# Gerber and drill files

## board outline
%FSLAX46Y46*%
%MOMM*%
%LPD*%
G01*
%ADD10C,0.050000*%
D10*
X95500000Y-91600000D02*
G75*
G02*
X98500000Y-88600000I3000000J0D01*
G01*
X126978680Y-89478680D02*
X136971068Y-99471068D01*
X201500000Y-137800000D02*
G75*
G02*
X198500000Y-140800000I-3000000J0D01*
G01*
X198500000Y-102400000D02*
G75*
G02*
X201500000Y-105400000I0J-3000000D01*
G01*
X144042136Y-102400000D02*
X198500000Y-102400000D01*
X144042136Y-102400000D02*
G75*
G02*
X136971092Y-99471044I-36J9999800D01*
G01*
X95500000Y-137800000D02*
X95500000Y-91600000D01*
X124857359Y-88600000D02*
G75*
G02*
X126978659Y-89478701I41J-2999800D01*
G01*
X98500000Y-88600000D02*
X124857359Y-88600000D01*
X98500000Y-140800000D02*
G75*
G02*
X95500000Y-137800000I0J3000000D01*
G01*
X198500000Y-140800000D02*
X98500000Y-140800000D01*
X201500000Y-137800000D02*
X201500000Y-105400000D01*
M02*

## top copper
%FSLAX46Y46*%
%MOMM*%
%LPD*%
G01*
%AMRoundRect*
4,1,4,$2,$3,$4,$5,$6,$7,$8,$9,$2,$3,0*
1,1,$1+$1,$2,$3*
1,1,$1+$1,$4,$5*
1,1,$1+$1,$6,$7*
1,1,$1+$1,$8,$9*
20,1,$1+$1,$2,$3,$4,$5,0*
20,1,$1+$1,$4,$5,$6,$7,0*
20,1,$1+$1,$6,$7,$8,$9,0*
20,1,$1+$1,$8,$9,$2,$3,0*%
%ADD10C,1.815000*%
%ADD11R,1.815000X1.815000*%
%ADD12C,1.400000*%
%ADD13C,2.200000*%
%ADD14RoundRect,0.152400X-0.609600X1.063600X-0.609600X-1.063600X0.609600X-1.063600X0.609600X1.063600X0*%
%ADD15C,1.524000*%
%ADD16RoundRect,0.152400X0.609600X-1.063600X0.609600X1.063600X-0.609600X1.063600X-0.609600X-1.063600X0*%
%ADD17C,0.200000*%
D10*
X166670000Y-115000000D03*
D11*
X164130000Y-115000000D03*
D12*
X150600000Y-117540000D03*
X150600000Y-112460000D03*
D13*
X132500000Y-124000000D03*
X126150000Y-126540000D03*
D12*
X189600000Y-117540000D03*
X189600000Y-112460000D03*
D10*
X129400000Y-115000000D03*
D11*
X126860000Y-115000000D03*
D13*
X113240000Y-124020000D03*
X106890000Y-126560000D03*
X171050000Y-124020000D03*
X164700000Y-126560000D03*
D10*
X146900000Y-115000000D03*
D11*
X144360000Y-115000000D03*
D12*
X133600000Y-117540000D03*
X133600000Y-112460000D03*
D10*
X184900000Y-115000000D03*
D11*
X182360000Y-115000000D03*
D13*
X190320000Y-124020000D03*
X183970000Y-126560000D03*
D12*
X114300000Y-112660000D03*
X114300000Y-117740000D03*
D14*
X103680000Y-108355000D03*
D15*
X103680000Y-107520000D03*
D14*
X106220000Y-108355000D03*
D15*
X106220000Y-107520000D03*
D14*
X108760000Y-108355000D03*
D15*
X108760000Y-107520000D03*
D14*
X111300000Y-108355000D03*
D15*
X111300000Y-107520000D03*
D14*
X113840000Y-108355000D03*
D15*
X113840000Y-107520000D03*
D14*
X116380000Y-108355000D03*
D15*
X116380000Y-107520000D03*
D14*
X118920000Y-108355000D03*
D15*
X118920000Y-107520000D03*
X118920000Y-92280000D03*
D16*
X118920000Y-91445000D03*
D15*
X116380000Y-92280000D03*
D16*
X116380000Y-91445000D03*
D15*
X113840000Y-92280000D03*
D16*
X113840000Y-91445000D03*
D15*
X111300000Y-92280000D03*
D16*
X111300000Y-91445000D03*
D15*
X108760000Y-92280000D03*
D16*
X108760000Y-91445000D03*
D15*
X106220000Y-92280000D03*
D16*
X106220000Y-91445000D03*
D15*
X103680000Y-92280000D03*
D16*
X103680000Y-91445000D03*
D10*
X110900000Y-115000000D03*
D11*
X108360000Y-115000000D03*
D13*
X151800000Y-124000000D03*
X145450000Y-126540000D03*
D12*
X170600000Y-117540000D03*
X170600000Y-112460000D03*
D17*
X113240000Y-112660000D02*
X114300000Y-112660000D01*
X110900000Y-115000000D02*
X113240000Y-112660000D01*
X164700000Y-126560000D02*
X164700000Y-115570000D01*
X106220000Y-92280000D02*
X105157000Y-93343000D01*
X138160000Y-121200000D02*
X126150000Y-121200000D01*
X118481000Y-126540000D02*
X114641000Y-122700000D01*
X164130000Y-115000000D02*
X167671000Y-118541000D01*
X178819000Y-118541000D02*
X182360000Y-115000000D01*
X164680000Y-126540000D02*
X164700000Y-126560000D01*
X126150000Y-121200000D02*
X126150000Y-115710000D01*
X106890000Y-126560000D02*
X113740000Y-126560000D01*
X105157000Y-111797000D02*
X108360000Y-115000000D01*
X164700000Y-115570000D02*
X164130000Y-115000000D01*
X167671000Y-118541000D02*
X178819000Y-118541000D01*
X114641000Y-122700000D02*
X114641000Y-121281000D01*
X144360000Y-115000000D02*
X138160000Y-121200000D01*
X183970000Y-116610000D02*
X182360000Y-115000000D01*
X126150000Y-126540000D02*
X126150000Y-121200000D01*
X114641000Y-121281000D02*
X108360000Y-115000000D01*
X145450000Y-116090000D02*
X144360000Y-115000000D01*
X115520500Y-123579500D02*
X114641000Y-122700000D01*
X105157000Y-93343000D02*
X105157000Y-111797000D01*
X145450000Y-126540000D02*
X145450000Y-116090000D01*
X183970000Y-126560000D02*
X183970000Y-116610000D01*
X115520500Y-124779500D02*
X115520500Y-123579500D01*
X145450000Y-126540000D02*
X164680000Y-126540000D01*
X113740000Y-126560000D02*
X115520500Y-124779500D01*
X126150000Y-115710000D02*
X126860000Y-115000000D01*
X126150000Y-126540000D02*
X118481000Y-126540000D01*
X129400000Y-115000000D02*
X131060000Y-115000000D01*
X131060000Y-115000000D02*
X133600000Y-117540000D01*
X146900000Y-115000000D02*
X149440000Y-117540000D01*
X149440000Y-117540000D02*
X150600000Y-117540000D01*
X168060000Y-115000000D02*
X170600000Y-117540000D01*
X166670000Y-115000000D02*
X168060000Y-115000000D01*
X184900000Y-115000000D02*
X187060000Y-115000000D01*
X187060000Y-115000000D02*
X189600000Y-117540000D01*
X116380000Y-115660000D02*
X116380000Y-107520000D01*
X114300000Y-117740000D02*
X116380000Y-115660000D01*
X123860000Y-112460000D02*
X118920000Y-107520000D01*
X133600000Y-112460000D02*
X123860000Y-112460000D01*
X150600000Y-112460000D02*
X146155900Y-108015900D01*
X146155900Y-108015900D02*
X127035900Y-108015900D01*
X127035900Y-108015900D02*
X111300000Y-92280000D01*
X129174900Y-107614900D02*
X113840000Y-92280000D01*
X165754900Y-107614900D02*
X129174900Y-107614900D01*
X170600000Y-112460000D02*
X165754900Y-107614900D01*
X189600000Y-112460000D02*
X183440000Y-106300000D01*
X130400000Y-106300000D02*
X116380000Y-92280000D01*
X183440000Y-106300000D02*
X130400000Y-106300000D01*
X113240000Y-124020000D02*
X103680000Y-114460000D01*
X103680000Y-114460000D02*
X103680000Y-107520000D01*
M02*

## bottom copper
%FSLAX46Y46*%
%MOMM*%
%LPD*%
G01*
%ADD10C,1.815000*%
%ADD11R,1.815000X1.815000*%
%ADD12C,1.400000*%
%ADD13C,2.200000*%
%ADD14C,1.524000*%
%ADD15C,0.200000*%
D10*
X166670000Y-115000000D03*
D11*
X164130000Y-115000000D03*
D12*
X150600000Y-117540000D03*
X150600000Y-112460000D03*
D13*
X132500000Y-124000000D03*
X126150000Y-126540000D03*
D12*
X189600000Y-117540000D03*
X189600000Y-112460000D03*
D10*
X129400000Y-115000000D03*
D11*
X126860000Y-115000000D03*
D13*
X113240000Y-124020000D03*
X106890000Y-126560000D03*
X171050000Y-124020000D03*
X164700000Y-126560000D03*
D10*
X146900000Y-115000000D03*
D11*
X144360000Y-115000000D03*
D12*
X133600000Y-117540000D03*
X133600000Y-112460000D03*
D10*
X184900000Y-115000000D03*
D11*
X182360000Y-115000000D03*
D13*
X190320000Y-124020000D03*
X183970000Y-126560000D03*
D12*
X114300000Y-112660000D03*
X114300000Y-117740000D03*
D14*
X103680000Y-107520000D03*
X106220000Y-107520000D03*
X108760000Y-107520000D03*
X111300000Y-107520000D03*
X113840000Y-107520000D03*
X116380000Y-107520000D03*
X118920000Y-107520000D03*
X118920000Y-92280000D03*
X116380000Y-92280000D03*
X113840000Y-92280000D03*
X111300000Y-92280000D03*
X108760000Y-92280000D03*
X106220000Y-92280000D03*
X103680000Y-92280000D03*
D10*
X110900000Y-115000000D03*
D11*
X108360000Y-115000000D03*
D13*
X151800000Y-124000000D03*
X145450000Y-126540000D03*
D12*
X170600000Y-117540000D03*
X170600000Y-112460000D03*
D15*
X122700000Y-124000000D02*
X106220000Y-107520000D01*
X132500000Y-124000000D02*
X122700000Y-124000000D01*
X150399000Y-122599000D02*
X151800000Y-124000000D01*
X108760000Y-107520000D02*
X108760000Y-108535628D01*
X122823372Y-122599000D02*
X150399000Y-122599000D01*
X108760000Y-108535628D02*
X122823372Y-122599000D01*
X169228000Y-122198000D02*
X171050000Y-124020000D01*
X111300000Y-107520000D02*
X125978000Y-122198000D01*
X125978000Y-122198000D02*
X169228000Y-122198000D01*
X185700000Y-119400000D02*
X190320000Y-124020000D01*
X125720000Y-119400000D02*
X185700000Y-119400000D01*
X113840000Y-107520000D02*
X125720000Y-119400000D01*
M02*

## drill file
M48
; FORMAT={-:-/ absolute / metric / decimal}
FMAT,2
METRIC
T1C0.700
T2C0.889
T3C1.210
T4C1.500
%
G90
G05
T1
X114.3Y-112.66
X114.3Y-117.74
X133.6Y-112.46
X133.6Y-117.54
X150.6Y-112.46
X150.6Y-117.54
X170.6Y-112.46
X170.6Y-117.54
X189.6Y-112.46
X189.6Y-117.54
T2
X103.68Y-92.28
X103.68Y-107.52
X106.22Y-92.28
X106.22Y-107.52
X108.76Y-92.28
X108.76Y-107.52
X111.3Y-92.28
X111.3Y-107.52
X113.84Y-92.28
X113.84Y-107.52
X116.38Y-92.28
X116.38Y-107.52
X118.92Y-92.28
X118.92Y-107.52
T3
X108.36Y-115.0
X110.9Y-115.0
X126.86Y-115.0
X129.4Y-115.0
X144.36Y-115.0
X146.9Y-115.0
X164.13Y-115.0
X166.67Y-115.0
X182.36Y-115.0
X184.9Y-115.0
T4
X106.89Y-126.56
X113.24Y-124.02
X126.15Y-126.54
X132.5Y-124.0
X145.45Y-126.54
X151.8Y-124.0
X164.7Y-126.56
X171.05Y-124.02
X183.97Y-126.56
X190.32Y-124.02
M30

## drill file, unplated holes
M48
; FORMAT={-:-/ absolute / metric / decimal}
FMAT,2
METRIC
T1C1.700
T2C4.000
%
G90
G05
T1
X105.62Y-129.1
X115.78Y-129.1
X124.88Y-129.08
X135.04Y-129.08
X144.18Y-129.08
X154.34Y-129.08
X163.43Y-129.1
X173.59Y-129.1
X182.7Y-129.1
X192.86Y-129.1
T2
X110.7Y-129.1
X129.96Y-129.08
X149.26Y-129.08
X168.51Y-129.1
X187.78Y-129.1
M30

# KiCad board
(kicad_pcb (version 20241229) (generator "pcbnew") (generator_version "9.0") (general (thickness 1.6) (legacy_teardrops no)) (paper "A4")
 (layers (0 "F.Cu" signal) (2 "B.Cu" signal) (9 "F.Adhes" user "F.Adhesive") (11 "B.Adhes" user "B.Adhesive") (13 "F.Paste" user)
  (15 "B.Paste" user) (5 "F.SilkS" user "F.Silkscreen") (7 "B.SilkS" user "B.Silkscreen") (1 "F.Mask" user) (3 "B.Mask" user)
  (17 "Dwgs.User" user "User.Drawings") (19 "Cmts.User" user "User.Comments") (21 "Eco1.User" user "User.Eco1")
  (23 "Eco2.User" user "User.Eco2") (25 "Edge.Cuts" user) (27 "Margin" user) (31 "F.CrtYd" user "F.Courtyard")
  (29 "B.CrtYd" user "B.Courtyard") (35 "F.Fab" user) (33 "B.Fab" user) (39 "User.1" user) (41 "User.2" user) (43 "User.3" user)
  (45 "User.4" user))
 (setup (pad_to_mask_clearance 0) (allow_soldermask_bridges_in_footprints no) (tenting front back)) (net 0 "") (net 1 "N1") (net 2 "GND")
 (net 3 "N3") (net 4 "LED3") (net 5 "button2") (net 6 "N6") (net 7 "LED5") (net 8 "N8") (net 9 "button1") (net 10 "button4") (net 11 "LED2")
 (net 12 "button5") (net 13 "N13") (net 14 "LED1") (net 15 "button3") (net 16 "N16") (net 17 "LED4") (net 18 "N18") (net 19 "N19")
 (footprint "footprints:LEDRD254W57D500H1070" (layer "F.Cu") (at 165.4 115)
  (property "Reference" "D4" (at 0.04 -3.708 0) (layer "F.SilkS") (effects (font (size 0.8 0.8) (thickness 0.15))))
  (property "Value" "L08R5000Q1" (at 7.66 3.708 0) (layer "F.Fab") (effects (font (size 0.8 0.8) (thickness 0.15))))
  (pad "A" thru_hole circle (at 1.27 0) (size 1.815 1.815) (drill 1.21) (layers "*.Cu" "*.Mask") (remove_unused_layers no) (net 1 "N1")
   (solder_mask_margin 0.102))
  (pad "C" thru_hole rect (at -1.27 0) (size 1.815 1.815) (drill 1.21) (layers "*.Cu" "*.Mask") (remove_unused_layers no) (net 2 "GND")
   (solder_mask_margin 0.102)))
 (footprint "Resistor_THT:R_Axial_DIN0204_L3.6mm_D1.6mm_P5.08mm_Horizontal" (layer "F.Cu") (at 150.6 117.54 90)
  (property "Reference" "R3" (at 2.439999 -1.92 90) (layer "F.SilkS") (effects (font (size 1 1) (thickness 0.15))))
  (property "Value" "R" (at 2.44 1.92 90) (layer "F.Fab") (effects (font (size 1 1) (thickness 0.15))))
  (pad "1" thru_hole circle (at 0 0 90) (size 1.4 1.4) (drill 0.7) (layers "*.Cu" "*.Mask") (remove_unused_layers no) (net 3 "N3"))
  (pad "2" thru_hole circle (at 5.08 0 90) (size 1.4 1.4) (drill 0.7) (layers "*.Cu" "*.Mask") (remove_unused_layers no) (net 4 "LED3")))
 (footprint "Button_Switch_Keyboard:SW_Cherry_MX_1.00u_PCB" (layer "F.Cu") (at 132.5 124)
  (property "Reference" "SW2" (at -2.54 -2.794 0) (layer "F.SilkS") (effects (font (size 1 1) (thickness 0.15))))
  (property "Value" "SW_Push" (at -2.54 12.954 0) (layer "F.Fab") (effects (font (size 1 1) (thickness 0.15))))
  (pad "" np_thru_hole circle (at -7.62 5.08) (size 1.7 1.7) (drill 1.7) (layers "*.Cu" "*.Mask"))
  (pad "" np_thru_hole circle (at -2.54 5.08) (size 4 4) (drill 4) (layers "*.Cu" "*.Mask"))
  (pad "" np_thru_hole circle (at 2.54 5.08) (size 1.7 1.7) (drill 1.7) (layers "*.Cu" "*.Mask"))
  (pad "1" thru_hole circle (at 0 0) (size 2.2 2.2) (drill 1.5) (layers "*.Cu" "*.Mask") (remove_unused_layers no) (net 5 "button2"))
  (pad "2" thru_hole circle (at -6.35 2.54) (size 2.2 2.2) (drill 1.5) (layers "*.Cu" "*.Mask") (remove_unused_layers no) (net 2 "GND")))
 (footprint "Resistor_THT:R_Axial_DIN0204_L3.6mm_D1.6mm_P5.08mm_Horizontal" (layer "F.Cu") (at 189.6 117.54 90)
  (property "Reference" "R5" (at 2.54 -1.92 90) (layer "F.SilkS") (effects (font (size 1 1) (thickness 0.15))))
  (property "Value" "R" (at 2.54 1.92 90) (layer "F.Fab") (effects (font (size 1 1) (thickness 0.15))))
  (pad "1" thru_hole circle (at 0 0 90) (size 1.4 1.4) (drill 0.7) (layers "*.Cu" "*.Mask") (remove_unused_layers no) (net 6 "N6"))
  (pad "2" thru_hole circle (at 5.08 0 90) (size 1.4 1.4) (drill 0.7) (layers "*.Cu" "*.Mask") (remove_unused_layers no) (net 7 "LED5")))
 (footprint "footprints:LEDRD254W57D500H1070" (layer "F.Cu") (at 128.13 115)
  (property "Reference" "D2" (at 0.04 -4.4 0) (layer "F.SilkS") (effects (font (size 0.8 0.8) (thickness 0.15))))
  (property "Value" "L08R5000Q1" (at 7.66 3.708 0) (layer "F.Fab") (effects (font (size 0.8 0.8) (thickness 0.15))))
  (pad "A" thru_hole circle (at 1.27 0) (size 1.815 1.815) (drill 1.21) (layers "*.Cu" "*.Mask") (remove_unused_layers no) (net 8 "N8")
   (solder_mask_margin 0.102))
  (pad "C" thru_hole rect (at -1.27 0) (size 1.815 1.815) (drill 1.21) (layers "*.Cu" "*.Mask") (remove_unused_layers no) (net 2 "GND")
   (solder_mask_margin 0.102)))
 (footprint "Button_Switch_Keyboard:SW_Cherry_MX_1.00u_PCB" (layer "F.Cu") (at 113.24 124.02)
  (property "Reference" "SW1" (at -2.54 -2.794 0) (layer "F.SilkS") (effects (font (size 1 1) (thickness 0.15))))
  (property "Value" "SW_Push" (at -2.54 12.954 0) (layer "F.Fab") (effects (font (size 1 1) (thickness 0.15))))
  (pad "" np_thru_hole circle (at -7.62 5.08) (size 1.7 1.7) (drill 1.7) (layers "*.Cu" "*.Mask"))
  (pad "" np_thru_hole circle (at -2.54 5.08) (size 4 4) (drill 4) (layers "*.Cu" "*.Mask"))
  (pad "" np_thru_hole circle (at 2.54 5.08) (size 1.7 1.7) (drill 1.7) (layers "*.Cu" "*.Mask"))
  (pad "1" thru_hole circle (at 0 0) (size 2.2 2.2) (drill 1.5) (layers "*.Cu" "*.Mask") (remove_unused_layers no) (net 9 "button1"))
  (pad "2" thru_hole circle (at -6.35 2.54) (size 2.2 2.2) (drill 1.5) (layers "*.Cu" "*.Mask") (remove_unused_layers no) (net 2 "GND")))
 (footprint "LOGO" (layer "F.Cu") (at 194.1 109.1)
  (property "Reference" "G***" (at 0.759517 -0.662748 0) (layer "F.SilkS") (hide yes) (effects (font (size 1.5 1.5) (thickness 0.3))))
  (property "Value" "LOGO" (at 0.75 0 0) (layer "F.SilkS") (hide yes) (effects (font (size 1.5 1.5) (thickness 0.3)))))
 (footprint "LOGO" (layer "F.Cu") (at 132.976092 101.625741 -30)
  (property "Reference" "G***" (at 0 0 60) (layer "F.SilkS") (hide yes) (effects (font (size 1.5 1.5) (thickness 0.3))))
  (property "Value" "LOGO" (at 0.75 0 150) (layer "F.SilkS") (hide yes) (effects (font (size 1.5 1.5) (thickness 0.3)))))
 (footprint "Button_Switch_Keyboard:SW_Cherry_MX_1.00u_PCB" (layer "F.Cu") (at 171.05 124.02)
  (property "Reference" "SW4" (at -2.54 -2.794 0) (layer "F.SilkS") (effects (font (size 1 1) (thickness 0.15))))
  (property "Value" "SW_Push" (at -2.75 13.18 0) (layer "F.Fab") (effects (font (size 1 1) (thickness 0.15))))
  (pad "" np_thru_hole circle (at -7.62 5.08) (size 1.7 1.7) (drill 1.7) (layers "*.Cu" "*.Mask"))
  (pad "" np_thru_hole circle (at -2.54 5.08) (size 4 4) (drill 4) (layers "*.Cu" "*.Mask"))
  (pad "" np_thru_hole circle (at 2.54 5.08) (size 1.7 1.7) (drill 1.7) (layers "*.Cu" "*.Mask"))
  (pad "1" thru_hole circle (at 0 0) (size 2.2 2.2) (drill 1.5) (layers "*.Cu" "*.Mask") (remove_unused_layers no) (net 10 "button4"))
  (pad "2" thru_hole circle (at -6.35 2.54) (size 2.2 2.2) (drill 1.5) (layers "*.Cu" "*.Mask") (remove_unused_layers no) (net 2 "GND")))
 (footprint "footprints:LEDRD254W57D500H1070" (layer "F.Cu") (at 145.63 115)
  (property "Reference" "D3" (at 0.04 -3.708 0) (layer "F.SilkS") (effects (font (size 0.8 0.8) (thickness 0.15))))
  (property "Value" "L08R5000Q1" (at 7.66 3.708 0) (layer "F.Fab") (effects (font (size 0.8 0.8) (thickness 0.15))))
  (pad "A" thru_hole circle (at 1.27 0) (size 1.815 1.815) (drill 1.21) (layers "*.Cu" "*.Mask") (remove_unused_layers no) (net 3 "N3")
   (solder_mask_margin 0.102))
  (pad "C" thru_hole rect (at -1.27 0) (size 1.815 1.815) (drill 1.21) (layers "*.Cu" "*.Mask") (remove_unused_layers no) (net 2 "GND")
   (solder_mask_margin 0.102)))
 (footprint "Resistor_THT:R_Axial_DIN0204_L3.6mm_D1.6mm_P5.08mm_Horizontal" (layer "F.Cu") (at 133.6 117.54 90)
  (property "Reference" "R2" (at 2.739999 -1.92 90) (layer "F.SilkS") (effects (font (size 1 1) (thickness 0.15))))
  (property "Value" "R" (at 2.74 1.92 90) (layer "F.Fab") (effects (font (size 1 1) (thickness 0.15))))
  (pad "1" thru_hole circle (at 0 0 90) (size 1.4 1.4) (drill 0.7) (layers "*.Cu" "*.Mask") (remove_unused_layers no) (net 8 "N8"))
  (pad "2" thru_hole circle (at 5.08 0 90) (size 1.4 1.4) (drill 0.7) (layers "*.Cu" "*.Mask") (remove_unused_layers no) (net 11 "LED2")))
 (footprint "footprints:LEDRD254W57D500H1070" (layer "F.Cu") (at 183.63 115)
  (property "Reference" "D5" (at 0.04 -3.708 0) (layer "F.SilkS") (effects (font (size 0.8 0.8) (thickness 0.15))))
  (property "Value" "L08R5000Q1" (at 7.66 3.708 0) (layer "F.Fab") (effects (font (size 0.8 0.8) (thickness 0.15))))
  (pad "A" thru_hole circle (at 1.27 0) (size 1.815 1.815) (drill 1.21) (layers "*.Cu" "*.Mask") (remove_unused_layers no) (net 6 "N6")
   (solder_mask_margin 0.102))
  (pad "C" thru_hole rect (at -1.27 0) (size 1.815 1.815) (drill 1.21) (layers "*.Cu" "*.Mask") (remove_unused_layers no) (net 2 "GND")
   (solder_mask_margin 0.102)))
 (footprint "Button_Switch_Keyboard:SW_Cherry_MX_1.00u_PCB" (layer "F.Cu") (at 190.32 124.02)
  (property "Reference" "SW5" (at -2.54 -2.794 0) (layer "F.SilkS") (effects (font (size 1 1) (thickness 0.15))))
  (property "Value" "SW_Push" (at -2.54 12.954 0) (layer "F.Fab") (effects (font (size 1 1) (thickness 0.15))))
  (pad "" np_thru_hole circle (at -7.62 5.08) (size 1.7 1.7) (drill 1.7) (layers "*.Cu" "*.Mask"))
  (pad "" np_thru_hole circle (at -2.54 5.08) (size 4 4) (drill 4) (layers "*.Cu" "*.Mask"))
  (pad "" np_thru_hole circle (at 2.54 5.08) (size 1.7 1.7) (drill 1.7) (layers "*.Cu" "*.Mask"))
  (pad "1" thru_hole circle (at 0 0) (size 2.2 2.2) (drill 1.5) (layers "*.Cu" "*.Mask") (remove_unused_layers no) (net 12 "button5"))
  (pad "2" thru_hole circle (at -6.35 2.54) (size 2.2 2.2) (drill 1.5) (layers "*.Cu" "*.Mask") (remove_unused_layers no) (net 2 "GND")))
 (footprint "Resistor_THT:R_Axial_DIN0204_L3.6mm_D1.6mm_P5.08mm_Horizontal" (layer "F.Cu") (at 114.3 112.66 -90)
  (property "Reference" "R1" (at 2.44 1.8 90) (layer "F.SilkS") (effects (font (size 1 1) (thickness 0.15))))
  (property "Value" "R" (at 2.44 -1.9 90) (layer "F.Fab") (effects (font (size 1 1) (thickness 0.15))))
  (pad "1" thru_hole circle (at 0 0 270) (size 1.4 1.4) (drill 0.7) (layers "*.Cu" "*.Mask") (remove_unused_layers no) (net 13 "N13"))
  (pad "2" thru_hole circle (at 5.08 0 270) (size 1.4 1.4) (drill 0.7) (layers "*.Cu" "*.Mask") (remove_unused_layers no) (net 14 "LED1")))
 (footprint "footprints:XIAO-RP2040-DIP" (layer "F.Cu") (at 111.3 99.9 90)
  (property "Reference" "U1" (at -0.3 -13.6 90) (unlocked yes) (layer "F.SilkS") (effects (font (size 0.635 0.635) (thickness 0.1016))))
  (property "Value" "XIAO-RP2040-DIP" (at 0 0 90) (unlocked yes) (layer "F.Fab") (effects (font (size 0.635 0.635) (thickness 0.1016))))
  (pad "1" smd roundrect (at -8.455 -7.62 270) (size 2.432 1.524) (layers "F.Cu" "F.Mask") (roundrect_rratio 0.1) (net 9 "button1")
   (thermal_bridge_angle 45))
  (pad "1" thru_hole circle (at -7.62 -7.62 270) (size 1.524 1.524) (drill 0.889) (layers "*.Cu" "*.Mask") (remove_unused_layers no)
   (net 9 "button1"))
  (pad "2" smd roundrect (at -8.455 -5.08 270) (size 2.432 1.524) (layers "F.Cu" "F.Mask") (roundrect_rratio 0.1) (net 5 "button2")
   (thermal_bridge_angle 45))
  (pad "2" thru_hole circle (at -7.62 -5.08 270) (size 1.524 1.524) (drill 0.889) (layers "*.Cu" "*.Mask") (remove_unused_layers no)
   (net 5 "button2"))
  (pad "3" smd roundrect (at -8.455 -2.54 270) (size 2.432 1.524) (layers "F.Cu" "F.Mask") (roundrect_rratio 0.1) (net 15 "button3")
   (thermal_bridge_angle 45))
  (pad "3" thru_hole circle (at -7.62 -2.54 270) (size 1.524 1.524) (drill 0.889) (layers "*.Cu" "*.Mask") (remove_unused_layers no)
   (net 15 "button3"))
  (pad "4" smd roundrect (at -8.455 0 270) (size 2.432 1.524) (layers "F.Cu" "F.Mask") (roundrect_rratio 0.1) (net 10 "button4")
   (thermal_bridge_angle 45))
  (pad "4" thru_hole circle (at -7.62 0 270) (size 1.524 1.524) (drill 0.889) (layers "*.Cu" "*.Mask") (remove_unused_layers no)
   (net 10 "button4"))
  (pad "5" smd roundrect (at -8.455 2.54 270) (size 2.432 1.524) (layers "F.Cu" "F.Mask") (roundrect_rratio 0.1) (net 12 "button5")
   (thermal_bridge_angle 45))
  (pad "5" thru_hole circle (at -7.62 2.54 270) (size 1.524 1.524) (drill 0.889) (layers "*.Cu" "*.Mask") (remove_unused_layers no)
   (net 12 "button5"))
  (pad "6" smd roundrect (at -8.455 5.08 270) (size 2.432 1.524) (layers "F.Cu" "F.Mask") (roundrect_rratio 0.1) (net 14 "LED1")
   (thermal_bridge_angle 45))
  (pad "6" thru_hole circle (at -7.62 5.08 270) (size 1.524 1.524) (drill 0.889) (layers "*.Cu" "*.Mask") (remove_unused_layers no)
   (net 14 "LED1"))
  (pad "7" smd roundrect (at -8.455 7.62 270) (size 2.432 1.524) (layers "F.Cu" "F.Mask") (roundrect_rratio 0.1) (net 11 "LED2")
   (thermal_bridge_angle 45))
  (pad "7" thru_hole circle (at -7.62 7.62 270) (size 1.524 1.524) (drill 0.889) (layers "*.Cu" "*.Mask") (remove_unused_layers no)
   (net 11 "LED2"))
  (pad "8" thru_hole circle (at 7.62 7.62 90) (size 1.524 1.524) (drill 0.889) (layers "*.Cu" "*.Mask") (remove_unused_layers no)
   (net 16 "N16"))
  (pad "8" smd roundrect (at 8.455 7.62 90) (size 2.432 1.524) (layers "F.Cu" "F.Mask") (roundrect_rratio 0.1) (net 16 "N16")
   (thermal_bridge_angle 45))
  (pad "9" thru_hole circle (at 7.62 5.08 90) (size 1.524 1.524) (drill 0.889) (layers "*.Cu" "*.Mask") (remove_unused_layers no)
   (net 7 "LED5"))
  (pad "9" smd roundrect (at 8.455 5.08 90) (size 2.432 1.524) (layers "F.Cu" "F.Mask") (roundrect_rratio 0.1) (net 7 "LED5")
   (thermal_bridge_angle 45))
  (pad "10" thru_hole circle (at 7.62 2.54 90) (size 1.524 1.524) (drill 0.889) (layers "*.Cu" "*.Mask") (remove_unused_layers no)
   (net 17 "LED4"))
  (pad "10" smd roundrect (at 8.455 2.54 90) (size 2.432 1.524) (layers "F.Cu" "F.Mask") (roundrect_rratio 0.1) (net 17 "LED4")
   (thermal_bridge_angle 45))
  (pad "11" thru_hole circle (at 7.62 0 90) (size 1.524 1.524) (drill 0.889) (layers "*.Cu" "*.Mask") (remove_unused_layers no)
   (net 4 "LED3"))
  (pad "11" smd roundrect (at 8.455 0 90) (size 2.432 1.524) (layers "F.Cu" "F.Mask") (roundrect_rratio 0.1) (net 4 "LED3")
   (thermal_bridge_angle 45))
  (pad "12" thru_hole circle (at 7.62 -2.54 90) (size 1.524 1.524) (drill 0.889) (layers "*.Cu" "*.Mask") (remove_unused_layers no)
   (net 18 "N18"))
  (pad "12" smd roundrect (at 8.455 -2.54 90) (size 2.432 1.524) (layers "F.Cu" "F.Mask") (roundrect_rratio 0.1) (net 18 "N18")
   (thermal_bridge_angle 45))
  (pad "13" thru_hole circle (at 7.62 -5.08 90) (size 1.524 1.524) (drill 0.889) (layers "*.Cu" "*.Mask") (remove_unused_layers no)
   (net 2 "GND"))
  (pad "13" smd roundrect (at 8.455 -5.08 90) (size 2.432 1.524) (layers "F.Cu" "F.Mask") (roundrect_rratio 0.1) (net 2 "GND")
   (thermal_bridge_angle 45))
  (pad "14" thru_hole circle (at 7.62 -7.62 90) (size 1.524 1.524) (drill 0.889) (layers "*.Cu" "*.Mask") (remove_unused_layers no)
   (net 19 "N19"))
  (pad "14" smd roundrect (at 8.455 -7.62 90) (size 2.432 1.524) (layers "F.Cu" "F.Mask") (roundrect_rratio 0.1) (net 19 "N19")
   (thermal_bridge_angle 45)))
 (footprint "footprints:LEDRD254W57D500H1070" (layer "F.Cu") (at 109.63 115)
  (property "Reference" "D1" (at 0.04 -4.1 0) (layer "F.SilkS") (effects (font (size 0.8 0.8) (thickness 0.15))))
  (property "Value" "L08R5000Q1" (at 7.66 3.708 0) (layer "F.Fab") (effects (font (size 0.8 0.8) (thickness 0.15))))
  (pad "A" thru_hole circle (at 1.27 0) (size 1.815 1.815) (drill 1.21) (layers "*.Cu" "*.Mask") (remove_unused_layers no) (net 13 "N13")
   (solder_mask_margin 0.102))
  (pad "C" thru_hole rect (at -1.27 0) (size 1.815 1.815) (drill 1.21) (layers "*.Cu" "*.Mask") (remove_unused_layers no) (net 2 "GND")
   (solder_mask_margin 0.102)))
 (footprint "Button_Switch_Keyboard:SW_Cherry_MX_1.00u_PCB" (layer "F.Cu") (at 151.8 124)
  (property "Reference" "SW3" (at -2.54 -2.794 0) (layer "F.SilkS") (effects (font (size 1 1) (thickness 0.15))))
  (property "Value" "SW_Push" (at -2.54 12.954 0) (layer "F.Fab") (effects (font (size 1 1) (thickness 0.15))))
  (pad "" np_thru_hole circle (at -7.62 5.08) (size 1.7 1.7) (drill 1.7) (layers "*.Cu" "*.Mask"))
  (pad "" np_thru_hole circle (at -2.54 5.08) (size 4 4) (drill 4) (layers "*.Cu" "*.Mask"))
  (pad "" np_thru_hole circle (at 2.54 5.08) (size 1.7 1.7) (drill 1.7) (layers "*.Cu" "*.Mask"))
  (pad "1" thru_hole circle (at 0 0) (size 2.2 2.2) (drill 1.5) (layers "*.Cu" "*.Mask") (remove_unused_layers no) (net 15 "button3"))
  (pad "2" thru_hole circle (at -6.35 2.54) (size 2.2 2.2) (drill 1.5) (layers "*.Cu" "*.Mask") (remove_unused_layers no) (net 2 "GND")))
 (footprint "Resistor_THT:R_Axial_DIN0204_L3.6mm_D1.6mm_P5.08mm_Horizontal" (layer "F.Cu") (at 170.6 117.54 90)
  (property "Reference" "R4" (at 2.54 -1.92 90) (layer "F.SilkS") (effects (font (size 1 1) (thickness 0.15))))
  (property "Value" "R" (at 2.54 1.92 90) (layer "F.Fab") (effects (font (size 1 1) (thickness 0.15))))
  (pad "1" thru_hole circle (at 0 0 90) (size 1.4 1.4) (drill 0.7) (layers "*.Cu" "*.Mask") (remove_unused_layers no) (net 1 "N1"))
  (pad "2" thru_hole circle (at 5.08 0 90) (size 1.4 1.4) (drill 0.7) (layers "*.Cu" "*.Mask") (remove_unused_layers no) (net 17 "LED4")))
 (gr_arc (start 95.5 91.6) (mid 96.37868 89.47868) (end 98.5 88.6) (stroke (width 0.05) (type default)) (layer "Edge.Cuts"))
 (gr_line (start 126.97868 89.47868) (end 136.971068 99.471068) (stroke (width 0.05) (type default)) (layer "Edge.Cuts"))
 (gr_arc (start 201.5 137.8) (mid 200.62132 139.92132) (end 198.5 140.8) (stroke (width 0.05) (type default)) (layer "Edge.Cuts"))
 (gr_arc (start 198.5 102.4) (mid 200.62132 103.27868) (end 201.5 105.4) (stroke (width 0.05) (type default)) (layer "Edge.Cuts"))
 (gr_line (start 144.042136 102.4) (end 198.5 102.4) (stroke (width 0.05) (type default)) (layer "Edge.Cuts"))
 (gr_arc (start 144.042136 102.4) (mid 140.215294 101.638807) (end 136.971068 99.471068) (stroke (width 0.05) (type default))
  (layer "Edge.Cuts"))
 (gr_line (start 95.5 137.8) (end 95.5 91.6) (stroke (width 0.05) (type default)) (layer "Edge.Cuts"))
 (gr_arc (start 124.857359 88.6) (mid 126.005418 88.828348) (end 126.97868 89.47868) (stroke (width 0.05) (type default))
  (layer "Edge.Cuts"))
 (gr_line (start 98.5 88.6) (end 124.857359 88.6) (stroke (width 0.05) (type default)) (layer "Edge.Cuts"))
 (gr_arc (start 98.5 140.8) (mid 96.37868 139.92132) (end 95.5 137.8) (stroke (width 0.05) (type default)) (layer "Edge.Cuts"))
 (gr_line (start 198.5 140.8) (end 98.5 140.8) (stroke (width 0.05) (type default)) (layer "Edge.Cuts"))
 (gr_line (start 201.5 137.8) (end 201.5 105.4) (stroke (width 0.05) (type default)) (layer "Edge.Cuts"))
 (segment (start 113.24 112.66) (end 114.3 112.66) (width 0.2) (layer "F.Cu") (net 13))
 (segment (start 110.9 115) (end 113.24 112.66) (width 0.2) (layer "F.Cu") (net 13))
 (segment (start 164.7 126.56) (end 164.7 115.57) (width 0.2) (layer "F.Cu") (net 2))
 (segment (start 106.22 92.28) (end 105.157 93.343) (width 0.2) (layer "F.Cu") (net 2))
 (segment (start 138.16 121.2) (end 126.15 121.2) (width 0.2) (layer "F.Cu") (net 2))
 (segment (start 118.481 126.54) (end 114.641 122.7) (width 0.2) (layer "F.Cu") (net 2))
 (segment (start 164.13 115) (end 167.671 118.541) (width 0.2) (layer "F.Cu") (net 2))
 (segment (start 178.819 118.541) (end 182.36 115) (width 0.2) (layer "F.Cu") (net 2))
 (segment (start 164.68 126.54) (end 164.7 126.56) (width 0.2) (layer "F.Cu") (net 2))
 (segment (start 126.15 121.2) (end 126.15 115.71) (width 0.2) (layer "F.Cu") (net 2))
 (segment (start 106.89 126.56) (end 113.74 126.56) (width 0.2) (layer "F.Cu") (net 2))
 (segment (start 105.157 111.797) (end 108.36 115) (width 0.2) (layer "F.Cu") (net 2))
 (segment (start 164.7 115.57) (end 164.13 115) (width 0.2) (layer "F.Cu") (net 2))
 (segment (start 167.671 118.541) (end 178.819 118.541) (width 0.2) (layer "F.Cu") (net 2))
 (segment (start 114.641 122.7) (end 114.641 121.281) (width 0.2) (layer "F.Cu") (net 2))
 (segment (start 144.36 115) (end 138.16 121.2) (width 0.2) (layer "F.Cu") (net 2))
 (segment (start 183.97 116.61) (end 182.36 115) (width 0.2) (layer "F.Cu") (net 2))
 (segment (start 126.15 126.54) (end 126.15 121.2) (width 0.2) (layer "F.Cu") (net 2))
 (segment (start 114.641 121.281) (end 108.36 115) (width 0.2) (layer "F.Cu") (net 2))
 (segment (start 145.45 116.09) (end 144.36 115) (width 0.2) (layer "F.Cu") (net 2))
 (segment (start 115.5205 123.5795) (end 114.641 122.7) (width 0.2) (layer "F.Cu") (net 2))
 (segment (start 105.157 93.343) (end 105.157 111.797) (width 0.2) (layer "F.Cu") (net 2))
 (segment (start 145.45 126.54) (end 145.45 116.09) (width 0.2) (layer "F.Cu") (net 2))
 (segment (start 183.97 126.56) (end 183.97 116.61) (width 0.2) (layer "F.Cu") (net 2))
 (segment (start 115.5205 124.7795) (end 115.5205 123.5795) (width 0.2) (layer "F.Cu") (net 2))
 (segment (start 145.45 126.54) (end 164.68 126.54) (width 0.2) (layer "F.Cu") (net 2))
 (segment (start 113.74 126.56) (end 115.5205 124.7795) (width 0.2) (layer "F.Cu") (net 2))
 (segment (start 126.15 115.71) (end 126.86 115) (width 0.2) (layer "F.Cu") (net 2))
 (segment (start 126.15 126.54) (end 118.481 126.54) (width 0.2) (layer "F.Cu") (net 2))
 (segment (start 129.4 115) (end 131.06 115) (width 0.2) (layer "F.Cu") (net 8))
 (segment (start 131.06 115) (end 133.6 117.54) (width 0.2) (layer "F.Cu") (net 8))
 (segment (start 146.9 115) (end 149.44 117.54) (width 0.2) (layer "F.Cu") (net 3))
 (segment (start 149.44 117.54) (end 150.6 117.54) (width 0.2) (layer "F.Cu") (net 3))
 (segment (start 168.06 115) (end 170.6 117.54) (width 0.2) (layer "F.Cu") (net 1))
 (segment (start 166.67 115) (end 168.06 115) (width 0.2) (layer "F.Cu") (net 1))
 (segment (start 184.9 115) (end 187.06 115) (width 0.2) (layer "F.Cu") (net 6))
 (segment (start 187.06 115) (end 189.6 117.54) (width 0.2) (layer "F.Cu") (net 6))
 (segment (start 116.38 115.66) (end 116.38 107.52) (width 0.2) (layer "F.Cu") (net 14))
 (segment (start 114.3 117.74) (end 116.38 115.66) (width 0.2) (layer "F.Cu") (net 14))
 (segment (start 123.86 112.46) (end 118.92 107.52) (width 0.2) (layer "F.Cu") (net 11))
 (segment (start 133.6 112.46) (end 123.86 112.46) (width 0.2) (layer "F.Cu") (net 11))
 (segment (start 150.6 112.46) (end 146.1559 108.0159) (width 0.2) (layer "F.Cu") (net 4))
 (segment (start 146.1559 108.0159) (end 127.0359 108.0159) (width 0.2) (layer "F.Cu") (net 4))
 (segment (start 127.0359 108.0159) (end 111.3 92.28) (width 0.2) (layer "F.Cu") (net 4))
 (segment (start 129.1749 107.6149) (end 113.84 92.28) (width 0.2) (layer "F.Cu") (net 17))
 (segment (start 165.7549 107.6149) (end 129.1749 107.6149) (width 0.2) (layer "F.Cu") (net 17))
 (segment (start 170.6 112.46) (end 165.7549 107.6149) (width 0.2) (layer "F.Cu") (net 17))
 (segment (start 189.6 112.46) (end 183.44 106.3) (width 0.2) (layer "F.Cu") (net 7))
 (segment (start 130.4 106.3) (end 116.38 92.28) (width 0.2) (layer "F.Cu") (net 7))
 (segment (start 183.44 106.3) (end 130.4 106.3) (width 0.2) (layer "F.Cu") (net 7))
 (segment (start 113.24 124.02) (end 103.68 114.46) (width 0.2) (layer "F.Cu") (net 9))
 (segment (start 103.68 114.46) (end 103.68 107.52) (width 0.2) (layer "F.Cu") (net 9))
 (segment (start 122.7 124) (end 106.22 107.52) (width 0.2) (layer "B.Cu") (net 5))
 (segment (start 132.5 124) (end 122.7 124) (width 0.2) (layer "B.Cu") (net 5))
 (segment (start 150.399 122.599) (end 151.8 124) (width 0.2) (layer "B.Cu") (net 15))
 (segment (start 108.76 107.52) (end 108.76 108.535628) (width 0.2) (layer "B.Cu") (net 15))
 (segment (start 122.823372 122.599) (end 150.399 122.599) (width 0.2) (layer "B.Cu") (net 15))
 (segment (start 108.76 108.535628) (end 122.823372 122.599) (width 0.2) (layer "B.Cu") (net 15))
 (segment (start 169.228 122.198) (end 171.05 124.02) (width 0.2) (layer "B.Cu") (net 10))
 (segment (start 111.3 107.52) (end 125.978 122.198) (width 0.2) (layer "B.Cu") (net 10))
 (segment (start 125.978 122.198) (end 169.228 122.198) (width 0.2) (layer "B.Cu") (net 10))
 (segment (start 185.7 119.4) (end 190.32 124.02) (width 0.2) (layer "B.Cu") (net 12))
 (segment (start 125.72 119.4) (end 185.7 119.4) (width 0.2) (layer "B.Cu") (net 12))
 (segment (start 113.84 107.52) (end 125.72 119.4) (width 0.2) (layer "B.Cu") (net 12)))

